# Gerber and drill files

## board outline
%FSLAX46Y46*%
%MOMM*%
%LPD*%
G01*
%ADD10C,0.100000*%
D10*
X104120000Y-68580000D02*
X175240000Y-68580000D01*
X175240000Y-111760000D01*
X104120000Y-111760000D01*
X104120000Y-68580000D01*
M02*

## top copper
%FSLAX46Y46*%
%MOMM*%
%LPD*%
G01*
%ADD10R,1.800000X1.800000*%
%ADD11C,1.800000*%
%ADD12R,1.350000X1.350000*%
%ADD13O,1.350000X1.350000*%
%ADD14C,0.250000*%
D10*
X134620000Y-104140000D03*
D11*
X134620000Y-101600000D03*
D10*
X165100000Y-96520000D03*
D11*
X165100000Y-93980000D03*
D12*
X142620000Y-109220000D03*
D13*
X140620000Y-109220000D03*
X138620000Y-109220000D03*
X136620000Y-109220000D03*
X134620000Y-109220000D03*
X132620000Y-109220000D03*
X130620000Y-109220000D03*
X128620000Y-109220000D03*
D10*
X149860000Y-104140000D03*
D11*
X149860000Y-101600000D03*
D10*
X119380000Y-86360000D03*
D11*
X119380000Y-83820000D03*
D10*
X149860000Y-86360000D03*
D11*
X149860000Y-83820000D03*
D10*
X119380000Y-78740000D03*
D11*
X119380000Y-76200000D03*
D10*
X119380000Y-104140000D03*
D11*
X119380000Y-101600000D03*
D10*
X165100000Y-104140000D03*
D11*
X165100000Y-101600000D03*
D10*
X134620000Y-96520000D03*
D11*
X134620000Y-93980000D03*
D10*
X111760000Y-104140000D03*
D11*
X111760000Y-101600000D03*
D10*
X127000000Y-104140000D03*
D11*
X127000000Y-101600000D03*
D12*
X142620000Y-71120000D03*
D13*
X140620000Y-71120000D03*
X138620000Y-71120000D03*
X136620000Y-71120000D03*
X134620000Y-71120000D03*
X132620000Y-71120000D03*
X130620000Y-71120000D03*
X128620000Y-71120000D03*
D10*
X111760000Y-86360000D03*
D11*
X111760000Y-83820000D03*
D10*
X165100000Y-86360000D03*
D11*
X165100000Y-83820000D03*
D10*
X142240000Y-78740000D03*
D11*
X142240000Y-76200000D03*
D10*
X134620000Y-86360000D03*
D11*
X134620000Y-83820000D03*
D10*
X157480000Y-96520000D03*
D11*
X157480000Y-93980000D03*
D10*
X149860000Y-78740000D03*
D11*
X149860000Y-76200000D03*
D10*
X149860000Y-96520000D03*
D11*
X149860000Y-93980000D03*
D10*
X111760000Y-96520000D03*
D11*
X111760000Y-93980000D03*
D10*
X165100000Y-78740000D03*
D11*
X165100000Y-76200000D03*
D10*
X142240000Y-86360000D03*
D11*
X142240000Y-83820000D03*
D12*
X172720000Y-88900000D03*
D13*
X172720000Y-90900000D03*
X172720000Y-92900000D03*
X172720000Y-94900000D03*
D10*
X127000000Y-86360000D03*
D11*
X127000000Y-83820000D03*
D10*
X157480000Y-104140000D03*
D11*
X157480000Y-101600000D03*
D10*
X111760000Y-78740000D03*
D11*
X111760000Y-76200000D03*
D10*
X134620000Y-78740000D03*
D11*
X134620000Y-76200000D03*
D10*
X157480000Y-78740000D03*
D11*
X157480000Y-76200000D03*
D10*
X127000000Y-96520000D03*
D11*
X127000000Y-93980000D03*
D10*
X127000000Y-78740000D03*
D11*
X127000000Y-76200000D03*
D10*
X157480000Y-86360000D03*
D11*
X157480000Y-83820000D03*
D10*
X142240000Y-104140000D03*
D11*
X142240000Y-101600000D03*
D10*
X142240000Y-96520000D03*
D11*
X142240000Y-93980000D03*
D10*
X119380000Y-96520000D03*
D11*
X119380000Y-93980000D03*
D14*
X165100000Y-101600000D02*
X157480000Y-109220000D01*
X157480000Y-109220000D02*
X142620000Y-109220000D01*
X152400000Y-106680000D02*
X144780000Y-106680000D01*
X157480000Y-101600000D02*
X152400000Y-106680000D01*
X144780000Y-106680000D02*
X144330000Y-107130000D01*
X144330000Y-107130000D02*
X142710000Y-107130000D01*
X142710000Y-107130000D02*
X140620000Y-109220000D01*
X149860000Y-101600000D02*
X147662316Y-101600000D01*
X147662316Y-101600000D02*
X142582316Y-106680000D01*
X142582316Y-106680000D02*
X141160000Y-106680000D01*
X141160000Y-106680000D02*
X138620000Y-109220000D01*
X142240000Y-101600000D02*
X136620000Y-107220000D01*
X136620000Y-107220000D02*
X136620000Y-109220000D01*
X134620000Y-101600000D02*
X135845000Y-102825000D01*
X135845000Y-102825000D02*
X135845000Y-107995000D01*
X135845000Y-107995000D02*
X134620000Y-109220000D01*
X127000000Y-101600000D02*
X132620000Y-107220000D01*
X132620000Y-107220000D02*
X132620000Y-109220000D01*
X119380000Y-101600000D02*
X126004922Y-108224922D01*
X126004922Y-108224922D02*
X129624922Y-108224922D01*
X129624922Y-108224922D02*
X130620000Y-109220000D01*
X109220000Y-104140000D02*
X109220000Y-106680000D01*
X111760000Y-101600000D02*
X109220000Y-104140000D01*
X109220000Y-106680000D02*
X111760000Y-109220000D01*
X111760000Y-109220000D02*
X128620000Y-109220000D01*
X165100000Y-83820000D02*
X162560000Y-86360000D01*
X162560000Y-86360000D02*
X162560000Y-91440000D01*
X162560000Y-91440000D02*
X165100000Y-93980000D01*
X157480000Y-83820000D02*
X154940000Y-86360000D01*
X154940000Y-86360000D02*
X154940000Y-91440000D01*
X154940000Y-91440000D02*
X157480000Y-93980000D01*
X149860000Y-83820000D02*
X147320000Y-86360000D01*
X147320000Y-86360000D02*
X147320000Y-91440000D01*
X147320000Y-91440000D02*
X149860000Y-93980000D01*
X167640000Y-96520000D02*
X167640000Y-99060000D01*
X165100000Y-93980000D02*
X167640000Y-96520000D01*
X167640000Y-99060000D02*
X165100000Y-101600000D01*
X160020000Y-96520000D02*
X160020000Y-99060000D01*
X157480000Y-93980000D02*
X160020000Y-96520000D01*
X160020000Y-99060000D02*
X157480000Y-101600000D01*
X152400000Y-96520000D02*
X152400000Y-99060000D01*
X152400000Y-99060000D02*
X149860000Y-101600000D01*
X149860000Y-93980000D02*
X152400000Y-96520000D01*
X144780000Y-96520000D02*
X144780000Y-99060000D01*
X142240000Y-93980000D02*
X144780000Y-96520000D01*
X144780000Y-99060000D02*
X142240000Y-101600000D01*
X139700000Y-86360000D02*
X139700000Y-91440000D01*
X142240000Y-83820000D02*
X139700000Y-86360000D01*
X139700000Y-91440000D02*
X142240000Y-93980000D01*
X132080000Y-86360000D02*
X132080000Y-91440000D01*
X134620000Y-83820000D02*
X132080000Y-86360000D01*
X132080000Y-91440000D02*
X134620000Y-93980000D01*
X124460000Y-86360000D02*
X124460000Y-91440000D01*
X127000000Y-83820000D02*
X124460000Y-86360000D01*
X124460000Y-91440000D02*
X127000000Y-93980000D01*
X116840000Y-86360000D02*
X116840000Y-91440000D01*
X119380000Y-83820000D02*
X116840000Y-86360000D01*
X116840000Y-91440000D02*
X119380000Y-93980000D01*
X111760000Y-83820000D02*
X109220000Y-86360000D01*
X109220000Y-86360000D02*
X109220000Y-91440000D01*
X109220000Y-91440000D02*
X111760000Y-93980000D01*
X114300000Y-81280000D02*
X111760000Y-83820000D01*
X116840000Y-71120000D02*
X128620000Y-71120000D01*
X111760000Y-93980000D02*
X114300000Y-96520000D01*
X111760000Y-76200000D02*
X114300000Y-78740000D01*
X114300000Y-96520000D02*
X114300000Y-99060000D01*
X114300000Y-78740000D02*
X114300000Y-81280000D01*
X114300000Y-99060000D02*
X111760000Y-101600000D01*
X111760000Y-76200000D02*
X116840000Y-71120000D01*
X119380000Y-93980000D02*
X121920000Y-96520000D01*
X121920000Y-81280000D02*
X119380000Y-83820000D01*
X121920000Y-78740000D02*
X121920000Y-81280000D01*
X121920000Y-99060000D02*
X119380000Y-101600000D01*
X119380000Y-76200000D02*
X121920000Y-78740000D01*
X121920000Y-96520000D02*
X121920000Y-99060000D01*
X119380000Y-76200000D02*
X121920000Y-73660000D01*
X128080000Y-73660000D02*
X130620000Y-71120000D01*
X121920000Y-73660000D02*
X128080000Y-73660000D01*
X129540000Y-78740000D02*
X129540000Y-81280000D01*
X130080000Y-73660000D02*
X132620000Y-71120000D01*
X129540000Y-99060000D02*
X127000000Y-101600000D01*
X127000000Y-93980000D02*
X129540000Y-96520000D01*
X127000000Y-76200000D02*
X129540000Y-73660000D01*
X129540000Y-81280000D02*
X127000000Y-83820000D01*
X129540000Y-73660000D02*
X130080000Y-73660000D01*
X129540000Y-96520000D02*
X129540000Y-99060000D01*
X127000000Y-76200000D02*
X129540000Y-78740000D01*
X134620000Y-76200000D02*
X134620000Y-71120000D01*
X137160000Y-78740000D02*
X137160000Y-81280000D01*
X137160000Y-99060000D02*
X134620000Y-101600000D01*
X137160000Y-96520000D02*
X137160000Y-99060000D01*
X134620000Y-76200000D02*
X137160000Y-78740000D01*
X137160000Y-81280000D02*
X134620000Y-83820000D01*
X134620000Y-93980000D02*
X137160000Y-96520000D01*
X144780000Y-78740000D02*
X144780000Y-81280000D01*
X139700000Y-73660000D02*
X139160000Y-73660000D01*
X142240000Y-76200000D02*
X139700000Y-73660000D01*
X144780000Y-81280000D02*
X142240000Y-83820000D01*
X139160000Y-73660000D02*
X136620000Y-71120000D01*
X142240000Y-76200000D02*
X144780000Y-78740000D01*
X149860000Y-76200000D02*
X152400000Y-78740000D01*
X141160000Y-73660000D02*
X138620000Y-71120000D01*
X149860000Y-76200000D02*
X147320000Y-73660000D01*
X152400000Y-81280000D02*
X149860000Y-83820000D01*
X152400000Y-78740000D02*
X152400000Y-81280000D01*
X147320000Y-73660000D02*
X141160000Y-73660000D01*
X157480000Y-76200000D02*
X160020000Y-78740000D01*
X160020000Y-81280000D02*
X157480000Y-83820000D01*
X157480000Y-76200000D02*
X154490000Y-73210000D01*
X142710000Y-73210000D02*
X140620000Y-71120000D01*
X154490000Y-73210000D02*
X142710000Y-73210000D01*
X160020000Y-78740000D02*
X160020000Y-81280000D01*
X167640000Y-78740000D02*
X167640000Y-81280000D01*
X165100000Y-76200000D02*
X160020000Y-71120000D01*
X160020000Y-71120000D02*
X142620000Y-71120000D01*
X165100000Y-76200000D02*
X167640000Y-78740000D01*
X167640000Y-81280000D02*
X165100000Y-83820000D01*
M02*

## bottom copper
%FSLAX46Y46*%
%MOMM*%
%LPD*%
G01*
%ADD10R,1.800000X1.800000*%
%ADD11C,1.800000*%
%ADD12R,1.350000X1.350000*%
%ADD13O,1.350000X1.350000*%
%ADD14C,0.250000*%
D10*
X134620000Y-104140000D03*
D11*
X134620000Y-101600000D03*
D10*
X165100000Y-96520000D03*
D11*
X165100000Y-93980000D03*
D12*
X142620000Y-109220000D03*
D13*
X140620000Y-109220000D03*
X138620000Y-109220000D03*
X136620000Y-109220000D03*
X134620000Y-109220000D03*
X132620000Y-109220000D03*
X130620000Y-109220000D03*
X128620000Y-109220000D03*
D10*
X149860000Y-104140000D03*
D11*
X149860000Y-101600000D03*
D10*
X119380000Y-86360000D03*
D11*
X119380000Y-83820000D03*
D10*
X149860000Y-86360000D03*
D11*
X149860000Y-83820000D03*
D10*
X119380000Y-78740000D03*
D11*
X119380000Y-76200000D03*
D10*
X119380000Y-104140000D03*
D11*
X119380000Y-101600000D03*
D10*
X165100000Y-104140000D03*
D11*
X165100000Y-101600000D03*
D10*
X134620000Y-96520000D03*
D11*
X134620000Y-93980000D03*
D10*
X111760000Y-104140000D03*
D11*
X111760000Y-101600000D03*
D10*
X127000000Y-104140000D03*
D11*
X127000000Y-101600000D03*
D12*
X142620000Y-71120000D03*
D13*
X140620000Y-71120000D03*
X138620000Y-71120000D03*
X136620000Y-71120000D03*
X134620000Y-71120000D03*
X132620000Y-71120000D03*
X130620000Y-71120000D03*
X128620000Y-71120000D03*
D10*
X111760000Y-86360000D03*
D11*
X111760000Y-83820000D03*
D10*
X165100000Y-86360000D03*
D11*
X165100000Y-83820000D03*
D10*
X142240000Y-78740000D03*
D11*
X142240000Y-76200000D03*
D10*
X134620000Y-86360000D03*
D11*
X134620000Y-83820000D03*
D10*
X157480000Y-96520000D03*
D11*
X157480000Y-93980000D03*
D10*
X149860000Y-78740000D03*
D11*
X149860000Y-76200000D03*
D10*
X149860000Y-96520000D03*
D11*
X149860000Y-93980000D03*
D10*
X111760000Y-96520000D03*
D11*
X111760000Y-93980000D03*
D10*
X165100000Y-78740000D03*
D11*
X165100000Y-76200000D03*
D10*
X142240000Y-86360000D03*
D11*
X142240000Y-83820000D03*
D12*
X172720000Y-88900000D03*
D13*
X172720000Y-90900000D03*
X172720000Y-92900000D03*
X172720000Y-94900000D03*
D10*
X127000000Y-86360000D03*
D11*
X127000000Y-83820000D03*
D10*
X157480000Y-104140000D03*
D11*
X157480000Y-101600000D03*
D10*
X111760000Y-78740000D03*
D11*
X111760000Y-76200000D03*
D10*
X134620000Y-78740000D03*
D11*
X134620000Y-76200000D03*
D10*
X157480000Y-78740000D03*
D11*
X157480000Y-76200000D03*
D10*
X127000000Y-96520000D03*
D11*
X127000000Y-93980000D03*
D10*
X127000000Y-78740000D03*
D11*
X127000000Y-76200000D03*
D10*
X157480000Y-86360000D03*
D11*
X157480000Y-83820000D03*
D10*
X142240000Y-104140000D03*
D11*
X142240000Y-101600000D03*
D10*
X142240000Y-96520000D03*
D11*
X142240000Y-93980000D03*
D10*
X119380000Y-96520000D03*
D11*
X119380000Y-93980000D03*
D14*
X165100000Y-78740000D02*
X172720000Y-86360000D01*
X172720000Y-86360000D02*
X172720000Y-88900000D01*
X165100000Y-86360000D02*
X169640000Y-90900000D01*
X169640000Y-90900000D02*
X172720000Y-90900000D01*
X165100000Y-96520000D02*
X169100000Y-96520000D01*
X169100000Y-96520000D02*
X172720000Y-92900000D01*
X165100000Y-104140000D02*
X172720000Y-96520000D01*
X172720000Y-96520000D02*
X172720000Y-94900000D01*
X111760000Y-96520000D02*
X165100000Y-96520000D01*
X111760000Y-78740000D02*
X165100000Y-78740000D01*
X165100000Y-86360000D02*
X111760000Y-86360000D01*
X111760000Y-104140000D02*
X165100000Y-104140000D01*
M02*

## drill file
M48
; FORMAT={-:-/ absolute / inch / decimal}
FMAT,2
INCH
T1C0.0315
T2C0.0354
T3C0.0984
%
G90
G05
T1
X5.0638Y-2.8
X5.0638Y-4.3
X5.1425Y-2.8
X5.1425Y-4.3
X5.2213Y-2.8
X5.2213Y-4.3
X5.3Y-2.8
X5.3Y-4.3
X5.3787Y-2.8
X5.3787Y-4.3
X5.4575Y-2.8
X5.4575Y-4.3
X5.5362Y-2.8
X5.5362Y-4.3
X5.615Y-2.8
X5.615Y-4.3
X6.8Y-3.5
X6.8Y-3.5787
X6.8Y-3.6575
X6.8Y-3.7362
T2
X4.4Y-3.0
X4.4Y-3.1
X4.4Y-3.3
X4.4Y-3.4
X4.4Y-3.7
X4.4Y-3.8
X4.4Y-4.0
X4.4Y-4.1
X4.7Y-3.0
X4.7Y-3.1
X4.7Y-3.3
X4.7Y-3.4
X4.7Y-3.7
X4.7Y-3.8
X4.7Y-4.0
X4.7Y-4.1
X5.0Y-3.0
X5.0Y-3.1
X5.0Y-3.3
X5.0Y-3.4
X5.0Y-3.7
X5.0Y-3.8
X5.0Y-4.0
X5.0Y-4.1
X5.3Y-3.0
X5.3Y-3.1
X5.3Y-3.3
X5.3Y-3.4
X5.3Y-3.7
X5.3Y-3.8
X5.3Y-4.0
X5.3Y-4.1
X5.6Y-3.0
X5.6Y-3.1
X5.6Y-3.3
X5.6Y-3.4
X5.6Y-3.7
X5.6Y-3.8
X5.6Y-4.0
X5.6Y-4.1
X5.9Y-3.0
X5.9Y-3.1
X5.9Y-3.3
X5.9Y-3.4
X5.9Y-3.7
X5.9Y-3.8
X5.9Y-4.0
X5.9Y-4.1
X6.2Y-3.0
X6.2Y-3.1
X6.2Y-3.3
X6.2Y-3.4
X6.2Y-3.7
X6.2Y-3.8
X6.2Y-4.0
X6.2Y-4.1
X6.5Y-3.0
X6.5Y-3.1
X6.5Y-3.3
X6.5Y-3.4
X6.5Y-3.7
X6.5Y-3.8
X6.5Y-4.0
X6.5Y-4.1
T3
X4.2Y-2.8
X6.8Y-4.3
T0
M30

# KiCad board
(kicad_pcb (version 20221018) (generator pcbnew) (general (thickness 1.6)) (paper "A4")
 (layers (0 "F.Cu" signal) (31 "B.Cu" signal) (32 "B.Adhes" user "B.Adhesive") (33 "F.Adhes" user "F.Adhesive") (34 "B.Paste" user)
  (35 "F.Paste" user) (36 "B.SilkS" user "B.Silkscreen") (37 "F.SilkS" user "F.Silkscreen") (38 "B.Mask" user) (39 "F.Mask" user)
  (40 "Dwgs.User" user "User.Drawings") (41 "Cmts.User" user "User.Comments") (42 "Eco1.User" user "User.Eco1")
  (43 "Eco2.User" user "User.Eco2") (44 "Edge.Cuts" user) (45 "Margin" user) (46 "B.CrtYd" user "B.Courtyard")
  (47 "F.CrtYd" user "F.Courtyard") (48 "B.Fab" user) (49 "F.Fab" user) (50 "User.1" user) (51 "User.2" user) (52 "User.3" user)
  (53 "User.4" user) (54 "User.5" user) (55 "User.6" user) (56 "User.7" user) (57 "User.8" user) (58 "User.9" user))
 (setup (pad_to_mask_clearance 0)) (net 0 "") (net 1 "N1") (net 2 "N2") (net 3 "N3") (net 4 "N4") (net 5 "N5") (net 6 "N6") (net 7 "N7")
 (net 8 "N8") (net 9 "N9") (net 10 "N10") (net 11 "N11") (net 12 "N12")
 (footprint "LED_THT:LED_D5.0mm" (layer "F.Cu") (at 119.38 86.36 90)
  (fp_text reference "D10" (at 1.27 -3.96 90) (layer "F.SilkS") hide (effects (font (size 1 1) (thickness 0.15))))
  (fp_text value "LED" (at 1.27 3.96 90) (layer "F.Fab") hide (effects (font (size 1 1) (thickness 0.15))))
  (pad "1" thru_hole rect (at 0 0 90) (size 1.8 1.8) (drill 0.9) (layers "*.Cu" "*.Mask") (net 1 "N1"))
  (pad "2" thru_hole circle (at 2.54 0 90) (size 1.8 1.8) (drill 0.9) (layers "*.Cu" "*.Mask") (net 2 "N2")))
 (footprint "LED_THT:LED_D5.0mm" (layer "F.Cu") (at 149.86 86.36 90)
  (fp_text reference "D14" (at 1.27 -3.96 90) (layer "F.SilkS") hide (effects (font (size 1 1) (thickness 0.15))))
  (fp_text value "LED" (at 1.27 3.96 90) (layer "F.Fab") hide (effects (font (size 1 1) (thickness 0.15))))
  (pad "1" thru_hole rect (at 0 0 90) (size 1.8 1.8) (drill 0.9) (layers "*.Cu" "*.Mask") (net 1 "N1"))
  (pad "2" thru_hole circle (at 2.54 0 90) (size 1.8 1.8) (drill 0.9) (layers "*.Cu" "*.Mask") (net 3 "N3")))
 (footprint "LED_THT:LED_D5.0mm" (layer "F.Cu") (at 119.38 78.74 90)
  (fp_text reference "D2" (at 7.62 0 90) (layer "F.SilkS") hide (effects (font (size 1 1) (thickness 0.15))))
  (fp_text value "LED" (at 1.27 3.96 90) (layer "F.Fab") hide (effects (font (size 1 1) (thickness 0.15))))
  (pad "1" thru_hole rect (at 0 0 90) (size 1.8 1.8) (drill 0.9) (layers "*.Cu" "*.Mask") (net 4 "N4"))
  (pad "2" thru_hole circle (at 2.54 0 90) (size 1.8 1.8) (drill 0.9) (layers "*.Cu" "*.Mask") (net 2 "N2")))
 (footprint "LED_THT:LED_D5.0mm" (layer "F.Cu") (at 149.86 104.14 90)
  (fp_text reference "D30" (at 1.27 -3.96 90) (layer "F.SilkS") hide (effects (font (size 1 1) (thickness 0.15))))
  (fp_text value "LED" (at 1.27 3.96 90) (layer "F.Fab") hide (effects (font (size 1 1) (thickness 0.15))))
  (pad "1" thru_hole rect (at 0 0 90) (size 1.8 1.8) (drill 0.9) (layers "*.Cu" "*.Mask") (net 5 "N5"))
  (pad "2" thru_hole circle (at 2.54 0 90) (size 1.8 1.8) (drill 0.9) (layers "*.Cu" "*.Mask") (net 3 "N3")))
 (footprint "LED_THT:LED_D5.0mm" (layer "F.Cu") (at 119.38 104.14 90)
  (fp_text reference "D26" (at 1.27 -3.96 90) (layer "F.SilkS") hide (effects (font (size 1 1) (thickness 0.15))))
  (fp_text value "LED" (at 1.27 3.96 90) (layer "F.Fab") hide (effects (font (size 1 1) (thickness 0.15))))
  (pad "1" thru_hole rect (at 0 0 90) (size 1.8 1.8) (drill 0.9) (layers "*.Cu" "*.Mask") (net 5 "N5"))
  (pad "2" thru_hole circle (at 2.54 0 90) (size 1.8 1.8) (drill 0.9) (layers "*.Cu" "*.Mask") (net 2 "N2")))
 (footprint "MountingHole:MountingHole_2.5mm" (layer "F.Cu") (at 106.68 71.12)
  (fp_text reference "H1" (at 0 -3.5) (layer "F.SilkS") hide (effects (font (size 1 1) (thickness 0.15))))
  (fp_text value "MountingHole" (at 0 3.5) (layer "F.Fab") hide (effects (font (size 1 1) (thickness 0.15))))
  (pad "" np_thru_hole circle (at 0 0) (size 2.5 2.5) (drill 2.5) (layers "*.Cu" "*.Mask")))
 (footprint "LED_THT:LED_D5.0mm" (layer "F.Cu") (at 165.1 104.14 90)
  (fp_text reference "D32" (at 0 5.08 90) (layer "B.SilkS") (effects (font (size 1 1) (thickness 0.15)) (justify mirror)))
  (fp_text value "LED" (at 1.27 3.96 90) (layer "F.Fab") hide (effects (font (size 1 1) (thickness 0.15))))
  (pad "1" thru_hole rect (at 0 0 90) (size 1.8 1.8) (drill 0.9) (layers "*.Cu" "*.Mask") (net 5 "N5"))
  (pad "2" thru_hole circle (at 2.54 0 90) (size 1.8 1.8) (drill 0.9) (layers "*.Cu" "*.Mask") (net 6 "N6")))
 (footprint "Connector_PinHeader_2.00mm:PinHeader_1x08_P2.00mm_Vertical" (layer "F.Cu") (at 142.62 109.22 -90)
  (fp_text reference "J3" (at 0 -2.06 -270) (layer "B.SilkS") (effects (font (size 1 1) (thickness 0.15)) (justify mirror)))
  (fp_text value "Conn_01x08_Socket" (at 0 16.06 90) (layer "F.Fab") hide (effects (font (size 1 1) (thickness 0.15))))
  (pad "1" thru_hole rect (at 0 0 270) (size 1.35 1.35) (drill 0.8) (layers "*.Cu" "*.Mask") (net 6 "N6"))
  (pad "2" thru_hole oval (at 0 2 270) (size 1.35 1.35) (drill 0.8) (layers "*.Cu" "*.Mask") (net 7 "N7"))
  (pad "3" thru_hole oval (at 0 4 270) (size 1.35 1.35) (drill 0.8) (layers "*.Cu" "*.Mask") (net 3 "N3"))
  (pad "4" thru_hole oval (at 0 6 270) (size 1.35 1.35) (drill 0.8) (layers "*.Cu" "*.Mask") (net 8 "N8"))
  (pad "5" thru_hole oval (at 0 8 270) (size 1.35 1.35) (drill 0.8) (layers "*.Cu" "*.Mask") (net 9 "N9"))
  (pad "6" thru_hole oval (at 0 10 270) (size 1.35 1.35) (drill 0.8) (layers "*.Cu" "*.Mask") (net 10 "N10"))
  (pad "7" thru_hole oval (at 0 12 270) (size 1.35 1.35) (drill 0.8) (layers "*.Cu" "*.Mask") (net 2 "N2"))
  (pad "8" thru_hole oval (at 0 14 270) (size 1.35 1.35) (drill 0.8) (layers "*.Cu" "*.Mask") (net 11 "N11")))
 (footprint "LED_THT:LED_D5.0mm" (layer "F.Cu") (at 134.62 96.52 90)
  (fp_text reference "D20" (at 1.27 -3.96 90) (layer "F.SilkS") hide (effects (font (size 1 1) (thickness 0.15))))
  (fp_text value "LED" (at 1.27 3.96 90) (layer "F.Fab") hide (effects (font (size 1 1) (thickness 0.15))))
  (pad "1" thru_hole rect (at 0 0 90) (size 1.8 1.8) (drill 0.9) (layers "*.Cu" "*.Mask") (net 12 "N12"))
  (pad "2" thru_hole circle (at 2.54 0 90) (size 1.8 1.8) (drill 0.9) (layers "*.Cu" "*.Mask") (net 9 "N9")))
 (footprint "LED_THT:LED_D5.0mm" (layer "F.Cu") (at 111.76 104.14 90)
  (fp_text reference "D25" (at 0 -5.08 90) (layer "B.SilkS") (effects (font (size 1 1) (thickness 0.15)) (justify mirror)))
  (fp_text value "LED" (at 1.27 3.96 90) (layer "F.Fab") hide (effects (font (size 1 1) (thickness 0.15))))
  (pad "1" thru_hole rect (at 0 0 90) (size 1.8 1.8) (drill 0.9) (layers "*.Cu" "*.Mask") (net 5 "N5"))
  (pad "2" thru_hole circle (at 2.54 0 90) (size 1.8 1.8) (drill 0.9) (layers "*.Cu" "*.Mask") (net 11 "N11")))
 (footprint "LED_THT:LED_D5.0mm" (layer "F.Cu") (at 127 104.14 90)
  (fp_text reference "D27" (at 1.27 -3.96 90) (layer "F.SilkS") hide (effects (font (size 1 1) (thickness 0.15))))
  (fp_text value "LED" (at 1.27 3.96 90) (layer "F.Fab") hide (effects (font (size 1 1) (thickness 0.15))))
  (pad "1" thru_hole rect (at 0 0 90) (size 1.8 1.8) (drill 0.9) (layers "*.Cu" "*.Mask") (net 5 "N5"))
  (pad "2" thru_hole circle (at 2.54 0 90) (size 1.8 1.8) (drill 0.9) (layers "*.Cu" "*.Mask") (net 10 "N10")))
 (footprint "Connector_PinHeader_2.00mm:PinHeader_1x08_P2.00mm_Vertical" (layer "F.Cu") (at 142.62 71.12 -90)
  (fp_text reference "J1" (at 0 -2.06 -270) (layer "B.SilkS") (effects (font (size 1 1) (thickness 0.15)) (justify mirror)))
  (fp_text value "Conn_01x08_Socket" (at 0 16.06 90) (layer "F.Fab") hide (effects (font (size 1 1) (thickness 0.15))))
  (pad "1" thru_hole rect (at 0 0 270) (size 1.35 1.35) (drill 0.8) (layers "*.Cu" "*.Mask") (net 6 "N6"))
  (pad "2" thru_hole oval (at 0 2 270) (size 1.35 1.35) (drill 0.8) (layers "*.Cu" "*.Mask") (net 7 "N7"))
  (pad "3" thru_hole oval (at 0 4 270) (size 1.35 1.35) (drill 0.8) (layers "*.Cu" "*.Mask") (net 3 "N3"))
  (pad "4" thru_hole oval (at 0 6 270) (size 1.35 1.35) (drill 0.8) (layers "*.Cu" "*.Mask") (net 8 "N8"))
  (pad "5" thru_hole oval (at 0 8 270) (size 1.35 1.35) (drill 0.8) (layers "*.Cu" "*.Mask") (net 9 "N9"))
  (pad "6" thru_hole oval (at 0 10 270) (size 1.35 1.35) (drill 0.8) (layers "*.Cu" "*.Mask") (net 10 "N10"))
  (pad "7" thru_hole oval (at 0 12 270) (size 1.35 1.35) (drill 0.8) (layers "*.Cu" "*.Mask") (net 2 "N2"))
  (pad "8" thru_hole oval (at 0 14 270) (size 1.35 1.35) (drill 0.8) (layers "*.Cu" "*.Mask") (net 11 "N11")))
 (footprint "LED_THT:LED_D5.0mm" (layer "F.Cu") (at 111.76 86.36 90)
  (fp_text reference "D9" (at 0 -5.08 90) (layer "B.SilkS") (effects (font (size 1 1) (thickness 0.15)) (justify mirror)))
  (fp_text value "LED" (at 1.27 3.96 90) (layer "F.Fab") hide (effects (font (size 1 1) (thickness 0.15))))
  (pad "1" thru_hole rect (at 0 0 90) (size 1.8 1.8) (drill 0.9) (layers "*.Cu" "*.Mask") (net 1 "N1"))
  (pad "2" thru_hole circle (at 2.54 0 90) (size 1.8 1.8) (drill 0.9) (layers "*.Cu" "*.Mask") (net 11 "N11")))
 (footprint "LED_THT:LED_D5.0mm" (layer "F.Cu") (at 165.1 86.36 90)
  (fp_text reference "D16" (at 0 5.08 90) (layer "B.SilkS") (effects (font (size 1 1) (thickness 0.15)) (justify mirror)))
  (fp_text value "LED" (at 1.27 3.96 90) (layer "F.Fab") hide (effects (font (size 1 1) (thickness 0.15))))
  (pad "1" thru_hole rect (at 0 0 90) (size 1.8 1.8) (drill 0.9) (layers "*.Cu" "*.Mask") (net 1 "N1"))
  (pad "2" thru_hole circle (at 2.54 0 90) (size 1.8 1.8) (drill 0.9) (layers "*.Cu" "*.Mask") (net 6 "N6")))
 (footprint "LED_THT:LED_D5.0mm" (layer "F.Cu") (at 142.24 78.74 90)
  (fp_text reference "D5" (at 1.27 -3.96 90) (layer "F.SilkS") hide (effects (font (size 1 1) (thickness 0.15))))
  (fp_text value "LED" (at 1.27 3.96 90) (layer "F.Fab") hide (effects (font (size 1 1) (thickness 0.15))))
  (pad "1" thru_hole rect (at 0 0 90) (size 1.8 1.8) (drill 0.9) (layers "*.Cu" "*.Mask") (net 4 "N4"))
  (pad "2" thru_hole circle (at 2.54 0 90) (size 1.8 1.8) (drill 0.9) (layers "*.Cu" "*.Mask") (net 8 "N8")))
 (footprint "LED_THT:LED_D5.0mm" (layer "F.Cu") (at 134.62 86.36 90)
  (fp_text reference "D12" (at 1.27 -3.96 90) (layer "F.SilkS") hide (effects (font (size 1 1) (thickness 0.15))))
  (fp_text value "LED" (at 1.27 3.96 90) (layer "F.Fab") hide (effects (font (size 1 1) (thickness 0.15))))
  (pad "1" thru_hole rect (at 0 0 90) (size 1.8 1.8) (drill 0.9) (layers "*.Cu" "*.Mask") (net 1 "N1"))
  (pad "2" thru_hole circle (at 2.54 0 90) (size 1.8 1.8) (drill 0.9) (layers "*.Cu" "*.Mask") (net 9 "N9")))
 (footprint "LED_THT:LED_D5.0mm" (layer "F.Cu") (at 157.48 96.52 90)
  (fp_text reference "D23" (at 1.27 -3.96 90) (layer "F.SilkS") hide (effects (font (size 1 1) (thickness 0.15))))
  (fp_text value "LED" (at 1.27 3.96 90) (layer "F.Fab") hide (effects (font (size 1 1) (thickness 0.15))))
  (pad "1" thru_hole rect (at 0 0 90) (size 1.8 1.8) (drill 0.9) (layers "*.Cu" "*.Mask") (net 12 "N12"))
  (pad "2" thru_hole circle (at 2.54 0 90) (size 1.8 1.8) (drill 0.9) (layers "*.Cu" "*.Mask") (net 7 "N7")))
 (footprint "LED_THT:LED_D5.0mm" (layer "F.Cu") (at 149.86 78.74 90)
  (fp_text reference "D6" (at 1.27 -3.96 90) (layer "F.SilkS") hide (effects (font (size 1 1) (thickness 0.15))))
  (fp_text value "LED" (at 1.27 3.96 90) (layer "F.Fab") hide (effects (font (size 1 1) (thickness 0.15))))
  (pad "1" thru_hole rect (at 0 0 90) (size 1.8 1.8) (drill 0.9) (layers "*.Cu" "*.Mask") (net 4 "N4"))
  (pad "2" thru_hole circle (at 2.54 0 90) (size 1.8 1.8) (drill 0.9) (layers "*.Cu" "*.Mask") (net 3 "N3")))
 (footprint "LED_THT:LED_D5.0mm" (layer "F.Cu") (at 134.62 104.14 90)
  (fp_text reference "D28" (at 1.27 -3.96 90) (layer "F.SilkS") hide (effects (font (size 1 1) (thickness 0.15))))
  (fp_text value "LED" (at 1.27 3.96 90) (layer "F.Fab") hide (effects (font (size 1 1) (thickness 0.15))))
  (pad "1" thru_hole rect (at 0 0 90) (size 1.8 1.8) (drill 0.9) (layers "*.Cu" "*.Mask") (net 5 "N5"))
  (pad "2" thru_hole circle (at 2.54 0 90) (size 1.8 1.8) (drill 0.9) (layers "*.Cu" "*.Mask") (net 9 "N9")))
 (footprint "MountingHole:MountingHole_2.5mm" (layer "F.Cu") (at 172.72 109.22)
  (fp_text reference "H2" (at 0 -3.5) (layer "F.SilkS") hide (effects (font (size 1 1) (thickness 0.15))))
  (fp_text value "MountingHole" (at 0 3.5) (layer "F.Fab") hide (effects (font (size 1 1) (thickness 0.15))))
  (pad "" np_thru_hole circle (at 0 0) (size 2.5 2.5) (drill 2.5) (layers "*.Cu" "*.Mask")))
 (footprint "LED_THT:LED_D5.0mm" (layer "F.Cu") (at 149.86 96.52 90)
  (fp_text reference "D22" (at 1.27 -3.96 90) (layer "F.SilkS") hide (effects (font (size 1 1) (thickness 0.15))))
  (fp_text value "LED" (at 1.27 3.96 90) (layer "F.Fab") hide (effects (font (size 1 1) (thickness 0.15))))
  (pad "1" thru_hole rect (at 0 0 90) (size 1.8 1.8) (drill 0.9) (layers "*.Cu" "*.Mask") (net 12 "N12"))
  (pad "2" thru_hole circle (at 2.54 0 90) (size 1.8 1.8) (drill 0.9) (layers "*.Cu" "*.Mask") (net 3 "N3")))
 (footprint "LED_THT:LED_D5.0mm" (layer "F.Cu") (at 165.1 96.52 90)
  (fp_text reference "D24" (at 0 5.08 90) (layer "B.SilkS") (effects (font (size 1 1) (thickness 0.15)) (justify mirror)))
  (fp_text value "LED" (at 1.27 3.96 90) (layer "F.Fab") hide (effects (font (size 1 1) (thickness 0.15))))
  (pad "1" thru_hole rect (at 0 0 90) (size 1.8 1.8) (drill 0.9) (layers "*.Cu" "*.Mask") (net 12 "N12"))
  (pad "2" thru_hole circle (at 2.54 0 90) (size 1.8 1.8) (drill 0.9) (layers "*.Cu" "*.Mask") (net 6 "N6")))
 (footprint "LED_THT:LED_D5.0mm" (layer "F.Cu") (at 111.76 96.52 90)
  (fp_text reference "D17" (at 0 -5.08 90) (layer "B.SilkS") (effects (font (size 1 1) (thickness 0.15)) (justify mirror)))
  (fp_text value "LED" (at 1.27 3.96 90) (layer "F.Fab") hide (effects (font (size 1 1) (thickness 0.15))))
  (pad "1" thru_hole rect (at 0 0 90) (size 1.8 1.8) (drill 0.9) (layers "*.Cu" "*.Mask") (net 12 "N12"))
  (pad "2" thru_hole circle (at 2.54 0 90) (size 1.8 1.8) (drill 0.9) (layers "*.Cu" "*.Mask") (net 11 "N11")))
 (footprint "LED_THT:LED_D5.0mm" (layer "F.Cu") (at 165.1 78.74 90)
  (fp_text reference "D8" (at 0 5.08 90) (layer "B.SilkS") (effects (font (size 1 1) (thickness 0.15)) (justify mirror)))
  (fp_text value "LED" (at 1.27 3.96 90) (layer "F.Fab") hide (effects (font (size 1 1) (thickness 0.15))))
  (pad "1" thru_hole rect (at 0 0 90) (size 1.8 1.8) (drill 0.9) (layers "*.Cu" "*.Mask") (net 4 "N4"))
  (pad "2" thru_hole circle (at 2.54 0 90) (size 1.8 1.8) (drill 0.9) (layers "*.Cu" "*.Mask") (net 6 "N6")))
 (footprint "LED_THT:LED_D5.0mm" (layer "F.Cu") (at 142.24 86.36 90)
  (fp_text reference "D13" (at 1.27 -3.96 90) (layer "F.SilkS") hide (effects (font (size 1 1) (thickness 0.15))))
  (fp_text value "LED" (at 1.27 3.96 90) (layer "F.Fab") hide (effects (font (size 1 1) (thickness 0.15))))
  (pad "1" thru_hole rect (at 0 0 90) (size 1.8 1.8) (drill 0.9) (layers "*.Cu" "*.Mask") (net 1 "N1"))
  (pad "2" thru_hole circle (at 2.54 0 90) (size 1.8 1.8) (drill 0.9) (layers "*.Cu" "*.Mask") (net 8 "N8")))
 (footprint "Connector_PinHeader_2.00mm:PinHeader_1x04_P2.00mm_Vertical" (layer "F.Cu") (at 172.72 88.9)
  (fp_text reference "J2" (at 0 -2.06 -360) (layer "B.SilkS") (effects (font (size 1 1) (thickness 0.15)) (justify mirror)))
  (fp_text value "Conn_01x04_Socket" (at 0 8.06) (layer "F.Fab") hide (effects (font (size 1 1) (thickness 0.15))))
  (pad "1" thru_hole rect (at 0 0) (size 1.35 1.35) (drill 0.8) (layers "*.Cu" "*.Mask") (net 4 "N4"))
  (pad "2" thru_hole oval (at 0 2) (size 1.35 1.35) (drill 0.8) (layers "*.Cu" "*.Mask") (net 1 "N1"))
  (pad "3" thru_hole oval (at 0 4) (size 1.35 1.35) (drill 0.8) (layers "*.Cu" "*.Mask") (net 12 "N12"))
  (pad "4" thru_hole oval (at 0 6) (size 1.35 1.35) (drill 0.8) (layers "*.Cu" "*.Mask") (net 5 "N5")))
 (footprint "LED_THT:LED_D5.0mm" (layer "F.Cu") (at 127 86.36 90)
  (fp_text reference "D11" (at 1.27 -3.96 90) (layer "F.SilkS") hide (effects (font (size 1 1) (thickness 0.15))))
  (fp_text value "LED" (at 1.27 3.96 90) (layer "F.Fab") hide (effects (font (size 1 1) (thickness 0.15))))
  (pad "1" thru_hole rect (at 0 0 90) (size 1.8 1.8) (drill 0.9) (layers "*.Cu" "*.Mask") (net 1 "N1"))
  (pad "2" thru_hole circle (at 2.54 0 90) (size 1.8 1.8) (drill 0.9) (layers "*.Cu" "*.Mask") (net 10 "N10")))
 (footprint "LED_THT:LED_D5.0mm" (layer "F.Cu") (at 157.48 104.14 90)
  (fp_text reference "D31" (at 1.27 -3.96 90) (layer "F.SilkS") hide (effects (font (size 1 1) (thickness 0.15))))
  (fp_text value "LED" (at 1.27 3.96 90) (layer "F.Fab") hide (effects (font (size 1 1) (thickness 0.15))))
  (pad "1" thru_hole rect (at 0 0 90) (size 1.8 1.8) (drill 0.9) (layers "*.Cu" "*.Mask") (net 5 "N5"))
  (pad "2" thru_hole circle (at 2.54 0 90) (size 1.8 1.8) (drill 0.9) (layers "*.Cu" "*.Mask") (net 7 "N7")))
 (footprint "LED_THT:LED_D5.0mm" (layer "F.Cu") (at 111.76 78.74 90)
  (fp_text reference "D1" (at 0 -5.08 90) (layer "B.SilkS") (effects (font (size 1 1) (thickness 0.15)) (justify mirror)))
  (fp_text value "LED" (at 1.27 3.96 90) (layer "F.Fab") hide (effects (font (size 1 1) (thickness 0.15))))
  (pad "1" thru_hole rect (at 0 0 90) (size 1.8 1.8) (drill 0.9) (layers "*.Cu" "*.Mask") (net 4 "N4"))
  (pad "2" thru_hole circle (at 2.54 0 90) (size 1.8 1.8) (drill 0.9) (layers "*.Cu" "*.Mask") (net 11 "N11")))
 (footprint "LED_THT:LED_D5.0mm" (layer "F.Cu") (at 134.62 78.74 90)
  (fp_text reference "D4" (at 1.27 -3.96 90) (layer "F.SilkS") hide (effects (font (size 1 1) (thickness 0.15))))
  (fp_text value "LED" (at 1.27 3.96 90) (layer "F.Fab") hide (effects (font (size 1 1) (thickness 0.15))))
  (pad "1" thru_hole rect (at 0 0 90) (size 1.8 1.8) (drill 0.9) (layers "*.Cu" "*.Mask") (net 4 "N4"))
  (pad "2" thru_hole circle (at 2.54 0 90) (size 1.8 1.8) (drill 0.9) (layers "*.Cu" "*.Mask") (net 9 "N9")))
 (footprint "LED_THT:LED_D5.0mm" (layer "F.Cu") (at 157.48 78.74 90)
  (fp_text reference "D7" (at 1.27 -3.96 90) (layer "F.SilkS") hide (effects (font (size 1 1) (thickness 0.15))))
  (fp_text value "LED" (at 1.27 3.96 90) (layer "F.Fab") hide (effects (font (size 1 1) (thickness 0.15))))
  (pad "1" thru_hole rect (at 0 0 90) (size 1.8 1.8) (drill 0.9) (layers "*.Cu" "*.Mask") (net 4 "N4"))
  (pad "2" thru_hole circle (at 2.54 0 90) (size 1.8 1.8) (drill 0.9) (layers "*.Cu" "*.Mask") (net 7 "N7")))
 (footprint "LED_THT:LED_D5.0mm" (layer "F.Cu") (at 127 96.52 90)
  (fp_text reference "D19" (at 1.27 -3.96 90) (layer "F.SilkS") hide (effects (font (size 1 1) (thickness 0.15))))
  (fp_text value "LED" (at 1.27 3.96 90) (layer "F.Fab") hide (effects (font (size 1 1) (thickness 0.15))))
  (pad "1" thru_hole rect (at 0 0 90) (size 1.8 1.8) (drill 0.9) (layers "*.Cu" "*.Mask") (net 12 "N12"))
  (pad "2" thru_hole circle (at 2.54 0 90) (size 1.8 1.8) (drill 0.9) (layers "*.Cu" "*.Mask") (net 10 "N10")))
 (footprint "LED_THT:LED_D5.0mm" (layer "F.Cu") (at 127 78.74 90)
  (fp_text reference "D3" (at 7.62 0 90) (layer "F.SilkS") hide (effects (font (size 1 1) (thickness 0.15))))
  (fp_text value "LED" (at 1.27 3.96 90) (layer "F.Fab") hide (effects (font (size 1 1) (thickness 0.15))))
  (pad "1" thru_hole rect (at 0 0 90) (size 1.8 1.8) (drill 0.9) (layers "*.Cu" "*.Mask") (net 4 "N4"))
  (pad "2" thru_hole circle (at 2.54 0 90) (size 1.8 1.8) (drill 0.9) (layers "*.Cu" "*.Mask") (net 10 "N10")))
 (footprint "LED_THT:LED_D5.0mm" (layer "F.Cu") (at 157.48 86.36 90)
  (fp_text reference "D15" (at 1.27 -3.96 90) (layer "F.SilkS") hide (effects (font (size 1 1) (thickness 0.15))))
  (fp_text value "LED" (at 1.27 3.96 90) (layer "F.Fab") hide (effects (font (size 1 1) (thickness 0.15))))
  (pad "1" thru_hole rect (at 0 0 90) (size 1.8 1.8) (drill 0.9) (layers "*.Cu" "*.Mask") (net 1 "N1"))
  (pad "2" thru_hole circle (at 2.54 0 90) (size 1.8 1.8) (drill 0.9) (layers "*.Cu" "*.Mask") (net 7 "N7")))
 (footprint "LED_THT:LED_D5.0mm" (layer "F.Cu") (at 142.24 104.14 90)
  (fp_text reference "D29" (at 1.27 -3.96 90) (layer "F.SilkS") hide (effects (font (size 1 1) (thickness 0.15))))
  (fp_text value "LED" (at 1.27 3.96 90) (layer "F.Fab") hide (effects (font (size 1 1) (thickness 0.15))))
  (pad "1" thru_hole rect (at 0 0 90) (size 1.8 1.8) (drill 0.9) (layers "*.Cu" "*.Mask") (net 5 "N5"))
  (pad "2" thru_hole circle (at 2.54 0 90) (size 1.8 1.8) (drill 0.9) (layers "*.Cu" "*.Mask") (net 8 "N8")))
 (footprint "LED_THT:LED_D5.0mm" (layer "F.Cu") (at 142.24 96.52 90)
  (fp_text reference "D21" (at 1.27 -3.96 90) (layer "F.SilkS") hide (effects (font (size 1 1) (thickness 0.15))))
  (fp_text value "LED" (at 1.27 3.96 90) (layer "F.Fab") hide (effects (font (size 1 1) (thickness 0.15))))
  (pad "1" thru_hole rect (at 0 0 90) (size 1.8 1.8) (drill 0.9) (layers "*.Cu" "*.Mask") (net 12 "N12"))
  (pad "2" thru_hole circle (at 2.54 0 90) (size 1.8 1.8) (drill 0.9) (layers "*.Cu" "*.Mask") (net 8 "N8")))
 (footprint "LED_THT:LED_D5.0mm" (layer "F.Cu") (at 119.38 96.52 90)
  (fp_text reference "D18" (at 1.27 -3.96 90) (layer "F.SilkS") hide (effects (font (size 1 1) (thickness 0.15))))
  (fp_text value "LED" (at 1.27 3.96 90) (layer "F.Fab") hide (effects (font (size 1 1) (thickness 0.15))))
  (pad "1" thru_hole rect (at 0 0 90) (size 1.8 1.8) (drill 0.9) (layers "*.Cu" "*.Mask") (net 12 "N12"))
  (pad "2" thru_hole circle (at 2.54 0 90) (size 1.8 1.8) (drill 0.9) (layers "*.Cu" "*.Mask") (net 2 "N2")))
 (gr_rect (start 104.12 68.58) (end 175.24 111.76) (stroke (width 0.1) (type default)) (fill none) (layer "Edge.Cuts"))
 (segment (start 165.1 78.74) (end 172.72 86.36) (width 0.25) (layer "B.Cu") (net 4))
 (segment (start 111.76 78.74) (end 165.1 78.74) (width 0.25) (layer "B.Cu") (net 4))
 (segment (start 172.72 86.36) (end 172.72 88.9) (width 0.25) (layer "B.Cu") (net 4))
 (segment (start 114.3 81.28) (end 111.76 83.82) (width 0.25) (layer "F.Cu") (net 11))
 (segment (start 116.84 71.12) (end 128.62 71.12) (width 0.25) (layer "F.Cu") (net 11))
 (segment (start 111.76 93.98) (end 114.3 96.52) (width 0.25) (layer "F.Cu") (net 11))
 (segment (start 109.22 106.68) (end 111.76 109.22) (width 0.25) (layer "F.Cu") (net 11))
 (segment (start 111.76 76.2) (end 114.3 78.74) (width 0.25) (layer "F.Cu") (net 11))
 (segment (start 109.22 91.44) (end 111.76 93.98) (width 0.25) (layer "F.Cu") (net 11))
 (segment (start 109.22 104.14) (end 109.22 106.68) (width 0.25) (layer "F.Cu") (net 11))
 (segment (start 109.22 86.36) (end 109.22 91.44) (width 0.25) (layer "F.Cu") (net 11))
 (segment (start 111.76 83.82) (end 109.22 86.36) (width 0.25) (layer "F.Cu") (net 11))
 (segment (start 114.3 96.52) (end 114.3 99.06) (width 0.25) (layer "F.Cu") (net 11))
 (segment (start 114.3 78.74) (end 114.3 81.28) (width 0.25) (layer "F.Cu") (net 11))
 (segment (start 114.3 99.06) (end 111.76 101.6) (width 0.25) (layer "F.Cu") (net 11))
 (segment (start 111.76 109.22) (end 128.62 109.22) (width 0.25) (layer "F.Cu") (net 11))
 (segment (start 111.76 76.2) (end 116.84 71.12) (width 0.25) (layer "F.Cu") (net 11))
 (segment (start 111.76 101.6) (end 109.22 104.14) (width 0.25) (layer "F.Cu") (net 11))
 (segment (start 126.004922 108.224922) (end 129.624922 108.224922) (width 0.25) (layer "F.Cu") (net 2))
 (segment (start 119.38 93.98) (end 121.92 96.52) (width 0.25) (layer "F.Cu") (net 2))
 (segment (start 129.624922 108.224922) (end 130.62 109.22) (width 0.25) (layer "F.Cu") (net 2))
 (segment (start 116.84 86.36) (end 116.84 91.44) (width 0.25) (layer "F.Cu") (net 2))
 (segment (start 116.84 91.44) (end 119.38 93.98) (width 0.25) (layer "F.Cu") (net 2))
 (segment (start 119.38 101.6) (end 126.004922 108.224922) (width 0.25) (layer "F.Cu") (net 2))
 (segment (start 121.92 81.28) (end 119.38 83.82) (width 0.25) (layer "F.Cu") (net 2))
 (segment (start 121.92 78.74) (end 121.92 81.28) (width 0.25) (layer "F.Cu") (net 2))
 (segment (start 121.92 99.06) (end 119.38 101.6) (width 0.25) (layer "F.Cu") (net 2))
 (segment (start 119.38 83.82) (end 116.84 86.36) (width 0.25) (layer "F.Cu") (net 2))
 (segment (start 119.38 76.2) (end 121.92 78.74) (width 0.25) (layer "F.Cu") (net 2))
 (segment (start 121.92 96.52) (end 121.92 99.06) (width 0.25) (layer "F.Cu") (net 2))
 (segment (start 119.38 76.2) (end 121.92 73.66) (width 0.25) (layer "F.Cu") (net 2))
 (segment (start 128.08 73.66) (end 130.62 71.12) (width 0.25) (layer "F.Cu") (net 2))
 (segment (start 121.92 73.66) (end 128.08 73.66) (width 0.25) (layer "F.Cu") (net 2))
 (segment (start 129.54 78.74) (end 129.54 81.28) (width 0.25) (layer "F.Cu") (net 10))
 (segment (start 130.08 73.66) (end 132.62 71.12) (width 0.25) (layer "F.Cu") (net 10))
 (segment (start 124.46 91.44) (end 127 93.98) (width 0.25) (layer "F.Cu") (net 10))
 (segment (start 129.54 99.06) (end 127 101.6) (width 0.25) (layer "F.Cu") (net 10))
 (segment (start 127 101.6) (end 132.62 107.22) (width 0.25) (layer "F.Cu") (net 10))
 (segment (start 124.46 86.36) (end 124.46 91.44) (width 0.25) (layer "F.Cu") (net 10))
 (segment (start 132.62 107.22) (end 132.62 109.22) (width 0.25) (layer "F.Cu") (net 10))
 (segment (start 127 93.98) (end 129.54 96.52) (width 0.25) (layer "F.Cu") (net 10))
 (segment (start 127 76.2) (end 129.54 73.66) (width 0.25) (layer "F.Cu") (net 10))
 (segment (start 127 83.82) (end 124.46 86.36) (width 0.25) (layer "F.Cu") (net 10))
 (segment (start 129.54 81.28) (end 127 83.82) (width 0.25) (layer "F.Cu") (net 10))
 (segment (start 129.54 73.66) (end 130.08 73.66) (width 0.25) (layer "F.Cu") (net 10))
 (segment (start 129.54 96.52) (end 129.54 99.06) (width 0.25) (layer "F.Cu") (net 10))
 (segment (start 127 76.2) (end 129.54 78.74) (width 0.25) (layer "F.Cu") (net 10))
 (segment (start 134.62 76.2) (end 134.62 71.12) (width 0.25) (layer "F.Cu") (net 9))
 (segment (start 135.845 102.825) (end 135.845 107.995) (width 0.25) (layer "F.Cu") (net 9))
 (segment (start 132.08 91.44) (end 134.62 93.98) (width 0.25) (layer "F.Cu") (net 9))
 (segment (start 134.62 83.82) (end 132.08 86.36) (width 0.25) (layer "F.Cu") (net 9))
 (segment (start 137.16 78.74) (end 137.16 81.28) (width 0.25) (layer "F.Cu") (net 9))
 (segment (start 134.62 101.6) (end 135.845 102.825) (width 0.25) (layer "F.Cu") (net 9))
 (segment (start 135.845 107.995) (end 134.62 109.22) (width 0.25) (layer "F.Cu") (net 9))
 (segment (start 137.16 99.06) (end 134.62 101.6) (width 0.25) (layer "F.Cu") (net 9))
 (segment (start 137.16 96.52) (end 137.16 99.06) (width 0.25) (layer "F.Cu") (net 9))
 (segment (start 134.62 76.2) (end 137.16 78.74) (width 0.25) (layer "F.Cu") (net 9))
 (segment (start 137.16 81.28) (end 134.62 83.82) (width 0.25) (layer "F.Cu") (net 9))
 (segment (start 134.62 93.98) (end 137.16 96.52) (width 0.25) (layer "F.Cu") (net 9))
 (segment (start 132.08 86.36) (end 132.08 91.44) (width 0.25) (layer "F.Cu") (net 9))
 (segment (start 144.78 78.74) (end 144.78 81.28) (width 0.25) (layer "F.Cu") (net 8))
 (segment (start 139.7 73.66) (end 139.16 73.66) (width 0.25) (layer "F.Cu") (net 8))
 (segment (start 142.24 76.2) (end 139.7 73.66) (width 0.25) (layer "F.Cu") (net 8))
 (segment (start 144.78 81.28) (end 142.24 83.82) (width 0.25) (layer "F.Cu") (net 8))
 (segment (start 139.16 73.66) (end 136.62 71.12) (width 0.25) (layer "F.Cu") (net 8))
 (segment (start 136.62 107.22) (end 136.62 109.22) (width 0.25) (layer "F.Cu") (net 8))
 (segment (start 142.24 93.98) (end 144.78 96.52) (width 0.25) (layer "F.Cu") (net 8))
 (segment (start 144.78 99.06) (end 142.24 101.6) (width 0.25) (layer "F.Cu") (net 8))
 (segment (start 144.78 96.52) (end 144.78 99.06) (width 0.25) (layer "F.Cu") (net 8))
 (segment (start 139.7 91.44) (end 142.24 93.98) (width 0.25) (layer "F.Cu") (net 8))
 (segment (start 142.24 101.6) (end 136.62 107.22) (width 0.25) (layer "F.Cu") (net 8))
 (segment (start 139.7 86.36) (end 139.7 91.44) (width 0.25) (layer "F.Cu") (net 8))
 (segment (start 142.24 76.2) (end 144.78 78.74) (width 0.25) (layer "F.Cu") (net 8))
 (segment (start 142.24 83.82) (end 139.7 86.36) (width 0.25) (layer "F.Cu") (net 8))
 (segment (start 147.32 86.36) (end 147.32 91.44) (width 0.25) (layer "F.Cu") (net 3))
 (segment (start 149.86 76.2) (end 152.4 78.74) (width 0.25) (layer "F.Cu") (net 3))
 (segment (start 141.16 73.66) (end 138.62 71.12) (width 0.25) (layer "F.Cu") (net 3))
 (segment (start 149.86 83.82) (end 147.32 86.36) (width 0.25) (layer "F.Cu") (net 3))
 (segment (start 149.86 101.6) (end 147.662316 101.6) (width 0.25) (layer "F.Cu") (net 3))
 (segment (start 147.662316 101.6) (end 142.582316 106.68) (width 0.25) (layer "F.Cu") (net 3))
 (segment (start 149.86 76.2) (end 147.32 73.66) (width 0.25) (layer "F.Cu") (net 3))
 (segment (start 152.4 99.06) (end 149.86 101.6) (width 0.25) (layer "F.Cu") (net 3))
 (segment (start 149.86 93.98) (end 152.4 96.52) (width 0.25) (layer "F.Cu") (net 3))
 (segment (start 152.4 81.28) (end 149.86 83.82) (width 0.25) (layer "F.Cu") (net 3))
 (segment (start 152.4 78.74) (end 152.4 81.28) (width 0.25) (layer "F.Cu") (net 3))
 (segment (start 147.32 91.44) (end 149.86 93.98) (width 0.25) (layer "F.Cu") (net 3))
 (segment (start 152.4 96.52) (end 152.4 99.06) (width 0.25) (layer "F.Cu") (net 3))
 (segment (start 142.582316 106.68) (end 141.16 106.68) (width 0.25) (layer "F.Cu") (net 3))
 (segment (start 147.32 73.66) (end 141.16 73.66) (width 0.25) (layer "F.Cu") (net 3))
 (segment (start 141.16 106.68) (end 138.62 109.22) (width 0.25) (layer "F.Cu") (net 3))
 (segment (start 157.48 76.2) (end 160.02 78.74) (width 0.25) (layer "F.Cu") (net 7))
 (segment (start 142.71 107.13) (end 140.62 109.22) (width 0.25) (layer "F.Cu") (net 7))
 (segment (start 160.02 81.28) (end 157.48 83.82) (width 0.25) (layer "F.Cu") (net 7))
 (segment (start 160.02 99.06) (end 157.48 101.6) (width 0.25) (layer "F.Cu") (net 7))
 (segment (start 144.33 107.13) (end 142.71 107.13) (width 0.25) (layer "F.Cu") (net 7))
 (segment (start 152.4 106.68) (end 144.78 106.68) (width 0.25) (layer "F.Cu") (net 7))
 (segment (start 157.48 76.2) (end 154.49 73.21) (width 0.25) (layer "F.Cu") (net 7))
 (segment (start 157.48 101.6) (end 152.4 106.68) (width 0.25) (layer "F.Cu") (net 7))
 (segment (start 142.71 73.21) (end 140.62 71.12) (width 0.25) (layer "F.Cu") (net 7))
 (segment (start 154.94 91.44) (end 157.48 93.98) (width 0.25) (layer "F.Cu") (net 7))
 (segment (start 144.78 106.68) (end 144.33 107.13) (width 0.25) (layer "F.Cu") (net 7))
 (segment (start 154.94 86.36) (end 154.94 91.44) (width 0.25) (layer "F.Cu") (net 7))
 (segment (start 154.49 73.21) (end 142.71 73.21) (width 0.25) (layer "F.Cu") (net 7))
 (segment (start 160.02 96.52) (end 160.02 99.06) (width 0.25) (layer "F.Cu") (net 7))
 (segment (start 157.48 93.98) (end 160.02 96.52) (width 0.25) (layer "F.Cu") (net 7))
 (segment (start 157.48 83.82) (end 154.94 86.36) (width 0.25) (layer "F.Cu") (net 7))
 (segment (start 160.02 78.74) (end 160.02 81.28) (width 0.25) (layer "F.Cu") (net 7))
 (segment (start 162.56 91.44) (end 165.1 93.98) (width 0.25) (layer "F.Cu") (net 6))
 (segment (start 167.64 78.74) (end 167.64 81.28) (width 0.25) (layer "F.Cu") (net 6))
 (segment (start 157.48 109.22) (end 142.62 109.22) (width 0.25) (layer "F.Cu") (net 6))
 (segment (start 165.1 83.82) (end 162.56 86.36) (width 0.25) (layer "F.Cu") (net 6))
 (segment (start 165.1 76.2) (end 160.02 71.12) (width 0.25) (layer "F.Cu") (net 6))
 (segment (start 165.1 93.98) (end 167.64 96.52) (width 0.25) (layer "F.Cu") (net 6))
 (segment (start 167.64 96.52) (end 167.64 99.06) (width 0.25) (layer "F.Cu") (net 6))
 (segment (start 162.56 86.36) (end 162.56 91.44) (width 0.25) (layer "F.Cu") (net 6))
 (segment (start 160.02 71.12) (end 142.62 71.12) (width 0.25) (layer "F.Cu") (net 6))
 (segment (start 165.1 76.2) (end 167.64 78.74) (width 0.25) (layer "F.Cu") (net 6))
 (segment (start 167.64 81.28) (end 165.1 83.82) (width 0.25) (layer "F.Cu") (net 6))
 (segment (start 167.64 99.06) (end 165.1 101.6) (width 0.25) (layer "F.Cu") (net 6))
 (segment (start 165.1 101.6) (end 157.48 109.22) (width 0.25) (layer "F.Cu") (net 6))
 (segment (start 165.1 86.36) (end 169.64 90.9) (width 0.25) (layer "B.Cu") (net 1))
 (segment (start 165.1 86.36) (end 111.76 86.36) (width 0.25) (layer "B.Cu") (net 1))
 (segment (start 169.64 90.9) (end 172.72 90.9) (width 0.25) (layer "B.Cu") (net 1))
 (segment (start 165.1 96.52) (end 169.1 96.52) (width 0.25) (layer "B.Cu") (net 12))
 (segment (start 111.76 96.52) (end 165.1 96.52) (width 0.25) (layer "B.Cu") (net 12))
 (segment (start 169.1 96.52) (end 172.72 92.9) (width 0.25) (layer "B.Cu") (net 12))
 (segment (start 165.1 104.14) (end 172.72 96.52) (width 0.25) (layer "B.Cu") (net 5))
 (segment (start 172.72 96.52) (end 172.72 94.9) (width 0.25) (layer "B.Cu") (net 5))
 (segment (start 111.76 104.14) (end 165.1 104.14) (width 0.25) (layer "B.Cu") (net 5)))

